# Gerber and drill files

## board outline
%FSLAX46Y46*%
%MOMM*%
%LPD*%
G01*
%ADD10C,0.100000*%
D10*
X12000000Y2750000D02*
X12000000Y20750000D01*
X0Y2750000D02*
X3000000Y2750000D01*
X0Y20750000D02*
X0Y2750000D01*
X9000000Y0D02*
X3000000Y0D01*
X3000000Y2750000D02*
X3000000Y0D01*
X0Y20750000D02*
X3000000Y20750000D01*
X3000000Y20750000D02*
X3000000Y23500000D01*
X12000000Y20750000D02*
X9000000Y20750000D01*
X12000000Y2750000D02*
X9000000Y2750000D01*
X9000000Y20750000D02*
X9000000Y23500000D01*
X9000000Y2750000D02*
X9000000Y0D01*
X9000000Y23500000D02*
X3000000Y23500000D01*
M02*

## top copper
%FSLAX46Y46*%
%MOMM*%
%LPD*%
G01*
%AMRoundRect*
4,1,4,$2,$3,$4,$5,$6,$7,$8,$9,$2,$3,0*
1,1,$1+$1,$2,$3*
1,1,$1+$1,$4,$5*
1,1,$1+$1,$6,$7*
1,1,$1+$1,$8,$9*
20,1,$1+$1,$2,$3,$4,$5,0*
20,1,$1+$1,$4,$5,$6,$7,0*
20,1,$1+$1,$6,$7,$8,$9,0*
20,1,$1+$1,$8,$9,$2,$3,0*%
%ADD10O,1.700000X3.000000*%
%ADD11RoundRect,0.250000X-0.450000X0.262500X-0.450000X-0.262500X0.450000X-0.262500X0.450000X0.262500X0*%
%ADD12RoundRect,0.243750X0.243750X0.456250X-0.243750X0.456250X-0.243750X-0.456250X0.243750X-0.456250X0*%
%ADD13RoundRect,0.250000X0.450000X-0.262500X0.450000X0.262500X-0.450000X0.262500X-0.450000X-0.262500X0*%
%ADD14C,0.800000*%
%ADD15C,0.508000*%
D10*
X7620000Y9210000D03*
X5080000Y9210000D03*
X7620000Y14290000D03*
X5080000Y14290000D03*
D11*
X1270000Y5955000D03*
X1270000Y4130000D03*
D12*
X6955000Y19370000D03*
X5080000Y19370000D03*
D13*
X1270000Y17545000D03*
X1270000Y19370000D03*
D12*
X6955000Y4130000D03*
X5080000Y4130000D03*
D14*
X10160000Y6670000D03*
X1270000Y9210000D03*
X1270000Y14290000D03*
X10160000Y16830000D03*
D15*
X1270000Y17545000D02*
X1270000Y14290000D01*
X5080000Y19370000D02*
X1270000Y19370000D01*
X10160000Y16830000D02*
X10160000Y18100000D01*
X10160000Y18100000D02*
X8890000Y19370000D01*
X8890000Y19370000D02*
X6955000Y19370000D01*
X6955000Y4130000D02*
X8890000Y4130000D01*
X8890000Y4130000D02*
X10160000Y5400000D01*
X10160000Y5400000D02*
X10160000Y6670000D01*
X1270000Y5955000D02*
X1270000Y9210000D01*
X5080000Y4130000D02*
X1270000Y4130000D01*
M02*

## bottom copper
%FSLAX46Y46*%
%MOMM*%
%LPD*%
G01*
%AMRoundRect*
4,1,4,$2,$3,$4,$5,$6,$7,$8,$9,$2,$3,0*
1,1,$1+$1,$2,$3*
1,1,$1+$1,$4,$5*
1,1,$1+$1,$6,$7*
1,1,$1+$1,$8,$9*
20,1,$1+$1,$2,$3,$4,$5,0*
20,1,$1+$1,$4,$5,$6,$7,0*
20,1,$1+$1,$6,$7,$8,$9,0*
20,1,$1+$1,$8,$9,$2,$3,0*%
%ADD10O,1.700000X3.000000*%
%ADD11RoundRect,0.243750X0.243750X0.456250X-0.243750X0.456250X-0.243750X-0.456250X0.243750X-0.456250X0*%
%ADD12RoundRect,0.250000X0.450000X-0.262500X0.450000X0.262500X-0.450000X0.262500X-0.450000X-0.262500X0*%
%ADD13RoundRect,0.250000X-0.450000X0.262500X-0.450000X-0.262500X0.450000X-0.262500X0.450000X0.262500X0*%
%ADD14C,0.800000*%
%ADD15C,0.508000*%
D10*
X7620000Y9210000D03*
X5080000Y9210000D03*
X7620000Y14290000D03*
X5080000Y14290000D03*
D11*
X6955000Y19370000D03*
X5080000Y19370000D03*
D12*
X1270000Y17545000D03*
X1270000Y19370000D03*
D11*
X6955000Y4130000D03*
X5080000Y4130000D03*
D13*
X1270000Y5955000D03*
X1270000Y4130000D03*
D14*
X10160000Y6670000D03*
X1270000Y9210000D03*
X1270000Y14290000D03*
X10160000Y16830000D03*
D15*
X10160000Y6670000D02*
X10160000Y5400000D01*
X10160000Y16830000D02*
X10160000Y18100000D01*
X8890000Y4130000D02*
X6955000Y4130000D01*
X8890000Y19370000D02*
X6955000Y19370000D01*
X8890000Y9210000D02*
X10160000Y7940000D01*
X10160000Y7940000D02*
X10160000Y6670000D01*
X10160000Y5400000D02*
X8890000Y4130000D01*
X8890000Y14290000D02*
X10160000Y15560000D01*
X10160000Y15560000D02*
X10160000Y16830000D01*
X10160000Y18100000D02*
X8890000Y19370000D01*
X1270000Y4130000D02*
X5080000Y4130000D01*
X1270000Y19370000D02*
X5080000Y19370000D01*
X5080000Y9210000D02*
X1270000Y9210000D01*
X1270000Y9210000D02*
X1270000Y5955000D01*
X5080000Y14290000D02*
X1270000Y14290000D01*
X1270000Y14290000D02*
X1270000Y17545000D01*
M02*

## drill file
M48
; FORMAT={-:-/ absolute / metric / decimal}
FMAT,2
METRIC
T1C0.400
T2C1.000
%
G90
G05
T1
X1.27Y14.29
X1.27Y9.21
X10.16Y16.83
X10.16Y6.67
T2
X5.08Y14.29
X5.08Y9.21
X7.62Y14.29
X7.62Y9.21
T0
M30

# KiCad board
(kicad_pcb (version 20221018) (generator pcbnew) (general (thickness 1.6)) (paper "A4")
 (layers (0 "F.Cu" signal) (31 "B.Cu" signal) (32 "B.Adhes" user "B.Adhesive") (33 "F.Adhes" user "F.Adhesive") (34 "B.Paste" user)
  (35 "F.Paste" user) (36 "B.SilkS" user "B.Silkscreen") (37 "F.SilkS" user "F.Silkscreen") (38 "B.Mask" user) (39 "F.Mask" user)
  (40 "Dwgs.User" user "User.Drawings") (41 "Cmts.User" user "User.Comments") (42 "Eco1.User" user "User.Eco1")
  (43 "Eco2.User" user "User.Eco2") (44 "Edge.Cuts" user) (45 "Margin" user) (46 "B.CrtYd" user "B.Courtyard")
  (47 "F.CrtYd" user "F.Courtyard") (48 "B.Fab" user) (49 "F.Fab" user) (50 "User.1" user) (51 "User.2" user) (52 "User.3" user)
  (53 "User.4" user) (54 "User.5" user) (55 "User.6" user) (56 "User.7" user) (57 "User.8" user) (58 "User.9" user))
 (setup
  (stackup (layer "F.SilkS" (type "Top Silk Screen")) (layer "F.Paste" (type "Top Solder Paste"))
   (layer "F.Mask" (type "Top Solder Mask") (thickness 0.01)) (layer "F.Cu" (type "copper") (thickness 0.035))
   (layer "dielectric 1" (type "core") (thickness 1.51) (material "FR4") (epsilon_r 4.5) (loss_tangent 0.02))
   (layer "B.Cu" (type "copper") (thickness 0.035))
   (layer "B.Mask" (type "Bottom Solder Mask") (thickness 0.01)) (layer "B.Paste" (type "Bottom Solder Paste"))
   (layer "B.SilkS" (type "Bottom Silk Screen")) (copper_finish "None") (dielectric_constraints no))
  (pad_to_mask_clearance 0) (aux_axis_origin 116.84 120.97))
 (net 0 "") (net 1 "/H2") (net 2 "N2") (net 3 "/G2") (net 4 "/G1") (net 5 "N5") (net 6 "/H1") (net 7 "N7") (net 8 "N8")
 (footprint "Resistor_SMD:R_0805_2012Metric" (layer "F.Cu") (at 118.11 115.9275 -90)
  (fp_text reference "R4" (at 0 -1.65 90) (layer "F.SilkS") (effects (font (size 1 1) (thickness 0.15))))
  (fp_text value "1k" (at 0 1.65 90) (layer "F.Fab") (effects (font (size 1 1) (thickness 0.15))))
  (pad "1" smd roundrect (at -0.9125 0 270) (size 1.025 1.4) (layers "F.Cu" "F.Paste" "F.Mask") (roundrect_rratio 0.243902439) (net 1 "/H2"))
  (pad "2" smd roundrect (at 0.9125 0 270) (size 1.025 1.4) (layers "F.Cu" "F.Paste" "F.Mask") (roundrect_rratio 0.243902439) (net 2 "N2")))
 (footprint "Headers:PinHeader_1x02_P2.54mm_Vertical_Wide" (layer "F.Cu") (at 124.46 111.76 -90)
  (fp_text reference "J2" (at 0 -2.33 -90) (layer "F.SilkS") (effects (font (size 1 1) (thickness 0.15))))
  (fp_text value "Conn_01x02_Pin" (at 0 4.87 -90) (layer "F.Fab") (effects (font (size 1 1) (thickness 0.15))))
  (pad "1" thru_hole oval (at 0 0 270) (size 3 1.7) (drill 1) (layers "*.Cu" "*.Mask") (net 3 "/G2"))
  (pad "2" thru_hole oval (at 0 2.54 270) (size 3 1.7) (drill 1) (layers "*.Cu" "*.Mask") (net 1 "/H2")))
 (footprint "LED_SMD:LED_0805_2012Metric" (layer "F.Cu") (at 122.8575 101.6 180)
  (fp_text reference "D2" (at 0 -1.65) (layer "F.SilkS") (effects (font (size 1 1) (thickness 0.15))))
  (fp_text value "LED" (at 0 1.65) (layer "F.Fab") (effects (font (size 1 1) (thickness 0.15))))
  (pad "1" smd roundrect (at -0.9375 0 180) (size 0.975 1.4) (layers "F.Cu" "F.Paste" "F.Mask") (roundrect_rratio 0.25) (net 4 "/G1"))
  (pad "2" smd roundrect (at 0.9375 0 180) (size 0.975 1.4) (layers "F.Cu" "F.Paste" "F.Mask") (roundrect_rratio 0.25) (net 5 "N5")))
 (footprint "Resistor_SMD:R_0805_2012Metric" (layer "F.Cu") (at 118.11 102.5125 90)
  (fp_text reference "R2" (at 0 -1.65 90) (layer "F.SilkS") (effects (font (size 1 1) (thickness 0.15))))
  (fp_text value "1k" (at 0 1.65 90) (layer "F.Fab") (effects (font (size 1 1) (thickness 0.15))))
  (pad "1" smd roundrect (at -0.9125 0 90) (size 1.025 1.4) (layers "F.Cu" "F.Paste" "F.Mask") (roundrect_rratio 0.243902439) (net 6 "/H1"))
  (pad "2" smd roundrect (at 0.9125 0 90) (size 1.025 1.4) (layers "F.Cu" "F.Paste" "F.Mask") (roundrect_rratio 0.243902439) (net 5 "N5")))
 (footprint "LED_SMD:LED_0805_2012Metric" (layer "F.Cu") (at 122.8575 116.84 180)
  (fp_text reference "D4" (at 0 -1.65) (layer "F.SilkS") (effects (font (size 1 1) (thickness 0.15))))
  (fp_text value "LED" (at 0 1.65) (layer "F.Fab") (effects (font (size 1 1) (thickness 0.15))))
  (pad "1" smd roundrect (at -0.9375 0 180) (size 0.975 1.4) (layers "F.Cu" "F.Paste" "F.Mask") (roundrect_rratio 0.25) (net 3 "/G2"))
  (pad "2" smd roundrect (at 0.9375 0 180) (size 0.975 1.4) (layers "F.Cu" "F.Paste" "F.Mask") (roundrect_rratio 0.25) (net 2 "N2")))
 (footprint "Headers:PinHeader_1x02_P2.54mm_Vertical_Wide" (layer "F.Cu") (at 124.46 106.68 -90)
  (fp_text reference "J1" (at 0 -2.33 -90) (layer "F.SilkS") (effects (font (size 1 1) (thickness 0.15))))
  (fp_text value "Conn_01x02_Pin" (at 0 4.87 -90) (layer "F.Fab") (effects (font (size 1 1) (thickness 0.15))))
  (pad "1" thru_hole oval (at 0 0 270) (size 3 1.7) (drill 1) (layers "*.Cu" "*.Mask") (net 4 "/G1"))
  (pad "2" thru_hole oval (at 0 2.54 270) (size 3 1.7) (drill 1) (layers "*.Cu" "*.Mask") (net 6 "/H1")))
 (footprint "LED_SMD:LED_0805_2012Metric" (layer "B.Cu") (at 122.8575 101.6 180)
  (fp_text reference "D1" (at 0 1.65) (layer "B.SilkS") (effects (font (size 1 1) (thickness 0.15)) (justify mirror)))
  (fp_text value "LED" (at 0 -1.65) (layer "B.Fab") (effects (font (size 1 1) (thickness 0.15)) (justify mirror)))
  (pad "1" smd roundrect (at -0.9375 0 180) (size 0.975 1.4) (layers "B.Cu" "B.Paste" "B.Mask") (roundrect_rratio 0.25) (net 4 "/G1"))
  (pad "2" smd roundrect (at 0.9375 0 180) (size 0.975 1.4) (layers "B.Cu" "B.Paste" "B.Mask") (roundrect_rratio 0.25) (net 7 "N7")))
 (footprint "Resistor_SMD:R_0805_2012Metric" (layer "B.Cu") (at 118.11 102.5125 90)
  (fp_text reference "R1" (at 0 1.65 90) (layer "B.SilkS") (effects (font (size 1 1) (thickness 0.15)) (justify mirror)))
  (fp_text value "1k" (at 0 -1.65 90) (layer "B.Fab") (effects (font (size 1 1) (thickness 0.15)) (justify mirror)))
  (pad "1" smd roundrect (at -0.9125 0 90) (size 1.025 1.4) (layers "B.Cu" "B.Paste" "B.Mask") (roundrect_rratio 0.243902439) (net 6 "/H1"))
  (pad "2" smd roundrect (at 0.9125 0 90) (size 1.025 1.4) (layers "B.Cu" "B.Paste" "B.Mask") (roundrect_rratio 0.243902439) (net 7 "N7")))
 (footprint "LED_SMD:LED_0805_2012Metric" (layer "B.Cu") (at 122.8575 116.84 180)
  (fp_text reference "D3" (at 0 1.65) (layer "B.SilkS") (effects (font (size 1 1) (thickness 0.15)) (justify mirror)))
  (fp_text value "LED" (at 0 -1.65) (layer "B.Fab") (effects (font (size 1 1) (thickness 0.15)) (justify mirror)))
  (pad "1" smd roundrect (at -0.9375 0 180) (size 0.975 1.4) (layers "B.Cu" "B.Paste" "B.Mask") (roundrect_rratio 0.25) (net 3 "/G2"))
  (pad "2" smd roundrect (at 0.9375 0 180) (size 0.975 1.4) (layers "B.Cu" "B.Paste" "B.Mask") (roundrect_rratio 0.25) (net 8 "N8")))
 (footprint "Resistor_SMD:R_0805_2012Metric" (layer "B.Cu") (at 118.11 115.9275 -90)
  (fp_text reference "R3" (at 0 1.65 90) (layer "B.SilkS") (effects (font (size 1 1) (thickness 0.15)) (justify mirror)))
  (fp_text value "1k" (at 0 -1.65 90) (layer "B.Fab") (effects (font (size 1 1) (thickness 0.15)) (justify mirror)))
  (pad "1" smd roundrect (at -0.9125 0 270) (size 1.025 1.4) (layers "B.Cu" "B.Paste" "B.Mask") (roundrect_rratio 0.243902439) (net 1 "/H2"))
  (pad "2" smd roundrect (at 0.9125 0 270) (size 1.025 1.4) (layers "B.Cu" "B.Paste" "B.Mask") (roundrect_rratio 0.243902439) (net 8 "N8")))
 (gr_line (start 128.84 118.22) (end 128.84 100.22) (stroke (width 0.1) (type default)) (layer "Edge.Cuts"))
 (gr_line (start 116.84 118.22) (end 119.84 118.22) (stroke (width 0.1) (type default)) (layer "Edge.Cuts"))
 (gr_line (start 116.84 100.22) (end 116.84 118.22) (stroke (width 0.1) (type default)) (layer "Edge.Cuts"))
 (gr_line (start 125.84 120.97) (end 119.84 120.97) (stroke (width 0.1) (type default)) (layer "Edge.Cuts"))
 (gr_line (start 119.84 118.22) (end 119.84 120.97) (stroke (width 0.1) (type default)) (layer "Edge.Cuts"))
 (gr_line (start 116.84 100.22) (end 119.84 100.22) (stroke (width 0.1) (type default)) (layer "Edge.Cuts"))
 (gr_line (start 119.84 100.22) (end 119.84 97.47) (stroke (width 0.1) (type default)) (layer "Edge.Cuts"))
 (gr_line (start 128.84 100.22) (end 125.84 100.22) (stroke (width 0.1) (type default)) (layer "Edge.Cuts"))
 (gr_line (start 128.84 118.22) (end 125.84 118.22) (stroke (width 0.1) (type default)) (layer "Edge.Cuts"))
 (gr_line (start 125.84 100.22) (end 125.84 97.47) (stroke (width 0.1) (type default)) (layer "Edge.Cuts"))
 (gr_line (start 125.84 118.22) (end 125.84 120.97) (stroke (width 0.1) (type default)) (layer "Edge.Cuts"))
 (gr_line (start 125.84 97.47) (end 119.84 97.47) (stroke (width 0.1) (type default)) (layer "Edge.Cuts"))
 (segment (start 118.11 101.6) (end 121.92 101.6) (width 0.508) (layer "B.Cu") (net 7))
 (segment (start 121.92 101.6) (end 118.11 101.6) (width 0.508) (layer "F.Cu") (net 5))
 (segment (start 118.11 116.84) (end 121.92 116.84) (width 0.508) (layer "B.Cu") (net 8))
 (segment (start 121.92 116.84) (end 118.11 116.84) (width 0.508) (layer "F.Cu") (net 2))
 (segment (start 125.73 101.6) (end 123.795 101.6) (width 0.508) (layer "F.Cu") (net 4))
 (segment (start 127 102.87) (end 125.73 101.6) (width 0.508) (layer "F.Cu") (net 4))
 (segment (start 127 104.14) (end 127 102.87) (width 0.508) (layer "F.Cu") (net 4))
 (via (at 127 104.14) (size 0.8) (drill 0.4) (layers "F.Cu" "B.Cu") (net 4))
 (segment (start 125.73 106.68) (end 127 105.41) (width 0.508) (layer "B.Cu") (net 4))
 (segment (start 127 104.14) (end 127 102.87) (width 0.508) (layer "B.Cu") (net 4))
 (segment (start 127 102.87) (end 125.73 101.6) (width 0.508) (layer "B.Cu") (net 4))
 (segment (start 125.73 101.6) (end 123.795 101.6) (width 0.508) (layer "B.Cu") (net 4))
 (segment (start 127 105.41) (end 127 104.14) (width 0.508) (layer "B.Cu") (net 4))
 (segment (start 125.73 116.84) (end 127 115.57) (width 0.508) (layer "F.Cu") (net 3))
 (segment (start 123.795 116.84) (end 125.73 116.84) (width 0.508) (layer "F.Cu") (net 3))
 (segment (start 127 115.57) (end 127 114.3) (width 0.508) (layer "F.Cu") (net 3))
 (via (at 127 114.3) (size 0.8) (drill 0.4) (layers "F.Cu" "B.Cu") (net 3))
 (segment (start 125.73 116.84) (end 123.795 116.84) (width 0.508) (layer "B.Cu") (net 3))
 (segment (start 127 115.57) (end 125.73 116.84) (width 0.508) (layer "B.Cu") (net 3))
 (segment (start 125.73 111.76) (end 127 113.03) (width 0.508) (layer "B.Cu") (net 3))
 (segment (start 127 113.03) (end 127 114.3) (width 0.508) (layer "B.Cu") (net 3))
 (segment (start 127 114.3) (end 127 115.57) (width 0.508) (layer "B.Cu") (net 3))
 (segment (start 118.11 103.425) (end 118.11 106.68) (width 0.508) (layer "F.Cu") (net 6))
 (via (at 118.11 106.68) (size 0.8) (drill 0.4) (layers "F.Cu" "B.Cu") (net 6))
 (segment (start 118.11 106.68) (end 118.11 103.425) (width 0.508) (layer "B.Cu") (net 6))
 (segment (start 121.92 106.68) (end 118.11 106.68) (width 0.508) (layer "B.Cu") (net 6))
 (segment (start 118.11 115.015) (end 118.11 111.76) (width 0.508) (layer "F.Cu") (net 1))
 (via (at 118.11 111.76) (size 0.8) (drill 0.4) (layers "F.Cu" "B.Cu") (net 1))
 (segment (start 121.92 111.76) (end 118.11 111.76) (width 0.508) (layer "B.Cu") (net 1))
 (segment (start 118.11 111.76) (end 118.11 115.015) (width 0.508) (layer "B.Cu") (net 1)))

